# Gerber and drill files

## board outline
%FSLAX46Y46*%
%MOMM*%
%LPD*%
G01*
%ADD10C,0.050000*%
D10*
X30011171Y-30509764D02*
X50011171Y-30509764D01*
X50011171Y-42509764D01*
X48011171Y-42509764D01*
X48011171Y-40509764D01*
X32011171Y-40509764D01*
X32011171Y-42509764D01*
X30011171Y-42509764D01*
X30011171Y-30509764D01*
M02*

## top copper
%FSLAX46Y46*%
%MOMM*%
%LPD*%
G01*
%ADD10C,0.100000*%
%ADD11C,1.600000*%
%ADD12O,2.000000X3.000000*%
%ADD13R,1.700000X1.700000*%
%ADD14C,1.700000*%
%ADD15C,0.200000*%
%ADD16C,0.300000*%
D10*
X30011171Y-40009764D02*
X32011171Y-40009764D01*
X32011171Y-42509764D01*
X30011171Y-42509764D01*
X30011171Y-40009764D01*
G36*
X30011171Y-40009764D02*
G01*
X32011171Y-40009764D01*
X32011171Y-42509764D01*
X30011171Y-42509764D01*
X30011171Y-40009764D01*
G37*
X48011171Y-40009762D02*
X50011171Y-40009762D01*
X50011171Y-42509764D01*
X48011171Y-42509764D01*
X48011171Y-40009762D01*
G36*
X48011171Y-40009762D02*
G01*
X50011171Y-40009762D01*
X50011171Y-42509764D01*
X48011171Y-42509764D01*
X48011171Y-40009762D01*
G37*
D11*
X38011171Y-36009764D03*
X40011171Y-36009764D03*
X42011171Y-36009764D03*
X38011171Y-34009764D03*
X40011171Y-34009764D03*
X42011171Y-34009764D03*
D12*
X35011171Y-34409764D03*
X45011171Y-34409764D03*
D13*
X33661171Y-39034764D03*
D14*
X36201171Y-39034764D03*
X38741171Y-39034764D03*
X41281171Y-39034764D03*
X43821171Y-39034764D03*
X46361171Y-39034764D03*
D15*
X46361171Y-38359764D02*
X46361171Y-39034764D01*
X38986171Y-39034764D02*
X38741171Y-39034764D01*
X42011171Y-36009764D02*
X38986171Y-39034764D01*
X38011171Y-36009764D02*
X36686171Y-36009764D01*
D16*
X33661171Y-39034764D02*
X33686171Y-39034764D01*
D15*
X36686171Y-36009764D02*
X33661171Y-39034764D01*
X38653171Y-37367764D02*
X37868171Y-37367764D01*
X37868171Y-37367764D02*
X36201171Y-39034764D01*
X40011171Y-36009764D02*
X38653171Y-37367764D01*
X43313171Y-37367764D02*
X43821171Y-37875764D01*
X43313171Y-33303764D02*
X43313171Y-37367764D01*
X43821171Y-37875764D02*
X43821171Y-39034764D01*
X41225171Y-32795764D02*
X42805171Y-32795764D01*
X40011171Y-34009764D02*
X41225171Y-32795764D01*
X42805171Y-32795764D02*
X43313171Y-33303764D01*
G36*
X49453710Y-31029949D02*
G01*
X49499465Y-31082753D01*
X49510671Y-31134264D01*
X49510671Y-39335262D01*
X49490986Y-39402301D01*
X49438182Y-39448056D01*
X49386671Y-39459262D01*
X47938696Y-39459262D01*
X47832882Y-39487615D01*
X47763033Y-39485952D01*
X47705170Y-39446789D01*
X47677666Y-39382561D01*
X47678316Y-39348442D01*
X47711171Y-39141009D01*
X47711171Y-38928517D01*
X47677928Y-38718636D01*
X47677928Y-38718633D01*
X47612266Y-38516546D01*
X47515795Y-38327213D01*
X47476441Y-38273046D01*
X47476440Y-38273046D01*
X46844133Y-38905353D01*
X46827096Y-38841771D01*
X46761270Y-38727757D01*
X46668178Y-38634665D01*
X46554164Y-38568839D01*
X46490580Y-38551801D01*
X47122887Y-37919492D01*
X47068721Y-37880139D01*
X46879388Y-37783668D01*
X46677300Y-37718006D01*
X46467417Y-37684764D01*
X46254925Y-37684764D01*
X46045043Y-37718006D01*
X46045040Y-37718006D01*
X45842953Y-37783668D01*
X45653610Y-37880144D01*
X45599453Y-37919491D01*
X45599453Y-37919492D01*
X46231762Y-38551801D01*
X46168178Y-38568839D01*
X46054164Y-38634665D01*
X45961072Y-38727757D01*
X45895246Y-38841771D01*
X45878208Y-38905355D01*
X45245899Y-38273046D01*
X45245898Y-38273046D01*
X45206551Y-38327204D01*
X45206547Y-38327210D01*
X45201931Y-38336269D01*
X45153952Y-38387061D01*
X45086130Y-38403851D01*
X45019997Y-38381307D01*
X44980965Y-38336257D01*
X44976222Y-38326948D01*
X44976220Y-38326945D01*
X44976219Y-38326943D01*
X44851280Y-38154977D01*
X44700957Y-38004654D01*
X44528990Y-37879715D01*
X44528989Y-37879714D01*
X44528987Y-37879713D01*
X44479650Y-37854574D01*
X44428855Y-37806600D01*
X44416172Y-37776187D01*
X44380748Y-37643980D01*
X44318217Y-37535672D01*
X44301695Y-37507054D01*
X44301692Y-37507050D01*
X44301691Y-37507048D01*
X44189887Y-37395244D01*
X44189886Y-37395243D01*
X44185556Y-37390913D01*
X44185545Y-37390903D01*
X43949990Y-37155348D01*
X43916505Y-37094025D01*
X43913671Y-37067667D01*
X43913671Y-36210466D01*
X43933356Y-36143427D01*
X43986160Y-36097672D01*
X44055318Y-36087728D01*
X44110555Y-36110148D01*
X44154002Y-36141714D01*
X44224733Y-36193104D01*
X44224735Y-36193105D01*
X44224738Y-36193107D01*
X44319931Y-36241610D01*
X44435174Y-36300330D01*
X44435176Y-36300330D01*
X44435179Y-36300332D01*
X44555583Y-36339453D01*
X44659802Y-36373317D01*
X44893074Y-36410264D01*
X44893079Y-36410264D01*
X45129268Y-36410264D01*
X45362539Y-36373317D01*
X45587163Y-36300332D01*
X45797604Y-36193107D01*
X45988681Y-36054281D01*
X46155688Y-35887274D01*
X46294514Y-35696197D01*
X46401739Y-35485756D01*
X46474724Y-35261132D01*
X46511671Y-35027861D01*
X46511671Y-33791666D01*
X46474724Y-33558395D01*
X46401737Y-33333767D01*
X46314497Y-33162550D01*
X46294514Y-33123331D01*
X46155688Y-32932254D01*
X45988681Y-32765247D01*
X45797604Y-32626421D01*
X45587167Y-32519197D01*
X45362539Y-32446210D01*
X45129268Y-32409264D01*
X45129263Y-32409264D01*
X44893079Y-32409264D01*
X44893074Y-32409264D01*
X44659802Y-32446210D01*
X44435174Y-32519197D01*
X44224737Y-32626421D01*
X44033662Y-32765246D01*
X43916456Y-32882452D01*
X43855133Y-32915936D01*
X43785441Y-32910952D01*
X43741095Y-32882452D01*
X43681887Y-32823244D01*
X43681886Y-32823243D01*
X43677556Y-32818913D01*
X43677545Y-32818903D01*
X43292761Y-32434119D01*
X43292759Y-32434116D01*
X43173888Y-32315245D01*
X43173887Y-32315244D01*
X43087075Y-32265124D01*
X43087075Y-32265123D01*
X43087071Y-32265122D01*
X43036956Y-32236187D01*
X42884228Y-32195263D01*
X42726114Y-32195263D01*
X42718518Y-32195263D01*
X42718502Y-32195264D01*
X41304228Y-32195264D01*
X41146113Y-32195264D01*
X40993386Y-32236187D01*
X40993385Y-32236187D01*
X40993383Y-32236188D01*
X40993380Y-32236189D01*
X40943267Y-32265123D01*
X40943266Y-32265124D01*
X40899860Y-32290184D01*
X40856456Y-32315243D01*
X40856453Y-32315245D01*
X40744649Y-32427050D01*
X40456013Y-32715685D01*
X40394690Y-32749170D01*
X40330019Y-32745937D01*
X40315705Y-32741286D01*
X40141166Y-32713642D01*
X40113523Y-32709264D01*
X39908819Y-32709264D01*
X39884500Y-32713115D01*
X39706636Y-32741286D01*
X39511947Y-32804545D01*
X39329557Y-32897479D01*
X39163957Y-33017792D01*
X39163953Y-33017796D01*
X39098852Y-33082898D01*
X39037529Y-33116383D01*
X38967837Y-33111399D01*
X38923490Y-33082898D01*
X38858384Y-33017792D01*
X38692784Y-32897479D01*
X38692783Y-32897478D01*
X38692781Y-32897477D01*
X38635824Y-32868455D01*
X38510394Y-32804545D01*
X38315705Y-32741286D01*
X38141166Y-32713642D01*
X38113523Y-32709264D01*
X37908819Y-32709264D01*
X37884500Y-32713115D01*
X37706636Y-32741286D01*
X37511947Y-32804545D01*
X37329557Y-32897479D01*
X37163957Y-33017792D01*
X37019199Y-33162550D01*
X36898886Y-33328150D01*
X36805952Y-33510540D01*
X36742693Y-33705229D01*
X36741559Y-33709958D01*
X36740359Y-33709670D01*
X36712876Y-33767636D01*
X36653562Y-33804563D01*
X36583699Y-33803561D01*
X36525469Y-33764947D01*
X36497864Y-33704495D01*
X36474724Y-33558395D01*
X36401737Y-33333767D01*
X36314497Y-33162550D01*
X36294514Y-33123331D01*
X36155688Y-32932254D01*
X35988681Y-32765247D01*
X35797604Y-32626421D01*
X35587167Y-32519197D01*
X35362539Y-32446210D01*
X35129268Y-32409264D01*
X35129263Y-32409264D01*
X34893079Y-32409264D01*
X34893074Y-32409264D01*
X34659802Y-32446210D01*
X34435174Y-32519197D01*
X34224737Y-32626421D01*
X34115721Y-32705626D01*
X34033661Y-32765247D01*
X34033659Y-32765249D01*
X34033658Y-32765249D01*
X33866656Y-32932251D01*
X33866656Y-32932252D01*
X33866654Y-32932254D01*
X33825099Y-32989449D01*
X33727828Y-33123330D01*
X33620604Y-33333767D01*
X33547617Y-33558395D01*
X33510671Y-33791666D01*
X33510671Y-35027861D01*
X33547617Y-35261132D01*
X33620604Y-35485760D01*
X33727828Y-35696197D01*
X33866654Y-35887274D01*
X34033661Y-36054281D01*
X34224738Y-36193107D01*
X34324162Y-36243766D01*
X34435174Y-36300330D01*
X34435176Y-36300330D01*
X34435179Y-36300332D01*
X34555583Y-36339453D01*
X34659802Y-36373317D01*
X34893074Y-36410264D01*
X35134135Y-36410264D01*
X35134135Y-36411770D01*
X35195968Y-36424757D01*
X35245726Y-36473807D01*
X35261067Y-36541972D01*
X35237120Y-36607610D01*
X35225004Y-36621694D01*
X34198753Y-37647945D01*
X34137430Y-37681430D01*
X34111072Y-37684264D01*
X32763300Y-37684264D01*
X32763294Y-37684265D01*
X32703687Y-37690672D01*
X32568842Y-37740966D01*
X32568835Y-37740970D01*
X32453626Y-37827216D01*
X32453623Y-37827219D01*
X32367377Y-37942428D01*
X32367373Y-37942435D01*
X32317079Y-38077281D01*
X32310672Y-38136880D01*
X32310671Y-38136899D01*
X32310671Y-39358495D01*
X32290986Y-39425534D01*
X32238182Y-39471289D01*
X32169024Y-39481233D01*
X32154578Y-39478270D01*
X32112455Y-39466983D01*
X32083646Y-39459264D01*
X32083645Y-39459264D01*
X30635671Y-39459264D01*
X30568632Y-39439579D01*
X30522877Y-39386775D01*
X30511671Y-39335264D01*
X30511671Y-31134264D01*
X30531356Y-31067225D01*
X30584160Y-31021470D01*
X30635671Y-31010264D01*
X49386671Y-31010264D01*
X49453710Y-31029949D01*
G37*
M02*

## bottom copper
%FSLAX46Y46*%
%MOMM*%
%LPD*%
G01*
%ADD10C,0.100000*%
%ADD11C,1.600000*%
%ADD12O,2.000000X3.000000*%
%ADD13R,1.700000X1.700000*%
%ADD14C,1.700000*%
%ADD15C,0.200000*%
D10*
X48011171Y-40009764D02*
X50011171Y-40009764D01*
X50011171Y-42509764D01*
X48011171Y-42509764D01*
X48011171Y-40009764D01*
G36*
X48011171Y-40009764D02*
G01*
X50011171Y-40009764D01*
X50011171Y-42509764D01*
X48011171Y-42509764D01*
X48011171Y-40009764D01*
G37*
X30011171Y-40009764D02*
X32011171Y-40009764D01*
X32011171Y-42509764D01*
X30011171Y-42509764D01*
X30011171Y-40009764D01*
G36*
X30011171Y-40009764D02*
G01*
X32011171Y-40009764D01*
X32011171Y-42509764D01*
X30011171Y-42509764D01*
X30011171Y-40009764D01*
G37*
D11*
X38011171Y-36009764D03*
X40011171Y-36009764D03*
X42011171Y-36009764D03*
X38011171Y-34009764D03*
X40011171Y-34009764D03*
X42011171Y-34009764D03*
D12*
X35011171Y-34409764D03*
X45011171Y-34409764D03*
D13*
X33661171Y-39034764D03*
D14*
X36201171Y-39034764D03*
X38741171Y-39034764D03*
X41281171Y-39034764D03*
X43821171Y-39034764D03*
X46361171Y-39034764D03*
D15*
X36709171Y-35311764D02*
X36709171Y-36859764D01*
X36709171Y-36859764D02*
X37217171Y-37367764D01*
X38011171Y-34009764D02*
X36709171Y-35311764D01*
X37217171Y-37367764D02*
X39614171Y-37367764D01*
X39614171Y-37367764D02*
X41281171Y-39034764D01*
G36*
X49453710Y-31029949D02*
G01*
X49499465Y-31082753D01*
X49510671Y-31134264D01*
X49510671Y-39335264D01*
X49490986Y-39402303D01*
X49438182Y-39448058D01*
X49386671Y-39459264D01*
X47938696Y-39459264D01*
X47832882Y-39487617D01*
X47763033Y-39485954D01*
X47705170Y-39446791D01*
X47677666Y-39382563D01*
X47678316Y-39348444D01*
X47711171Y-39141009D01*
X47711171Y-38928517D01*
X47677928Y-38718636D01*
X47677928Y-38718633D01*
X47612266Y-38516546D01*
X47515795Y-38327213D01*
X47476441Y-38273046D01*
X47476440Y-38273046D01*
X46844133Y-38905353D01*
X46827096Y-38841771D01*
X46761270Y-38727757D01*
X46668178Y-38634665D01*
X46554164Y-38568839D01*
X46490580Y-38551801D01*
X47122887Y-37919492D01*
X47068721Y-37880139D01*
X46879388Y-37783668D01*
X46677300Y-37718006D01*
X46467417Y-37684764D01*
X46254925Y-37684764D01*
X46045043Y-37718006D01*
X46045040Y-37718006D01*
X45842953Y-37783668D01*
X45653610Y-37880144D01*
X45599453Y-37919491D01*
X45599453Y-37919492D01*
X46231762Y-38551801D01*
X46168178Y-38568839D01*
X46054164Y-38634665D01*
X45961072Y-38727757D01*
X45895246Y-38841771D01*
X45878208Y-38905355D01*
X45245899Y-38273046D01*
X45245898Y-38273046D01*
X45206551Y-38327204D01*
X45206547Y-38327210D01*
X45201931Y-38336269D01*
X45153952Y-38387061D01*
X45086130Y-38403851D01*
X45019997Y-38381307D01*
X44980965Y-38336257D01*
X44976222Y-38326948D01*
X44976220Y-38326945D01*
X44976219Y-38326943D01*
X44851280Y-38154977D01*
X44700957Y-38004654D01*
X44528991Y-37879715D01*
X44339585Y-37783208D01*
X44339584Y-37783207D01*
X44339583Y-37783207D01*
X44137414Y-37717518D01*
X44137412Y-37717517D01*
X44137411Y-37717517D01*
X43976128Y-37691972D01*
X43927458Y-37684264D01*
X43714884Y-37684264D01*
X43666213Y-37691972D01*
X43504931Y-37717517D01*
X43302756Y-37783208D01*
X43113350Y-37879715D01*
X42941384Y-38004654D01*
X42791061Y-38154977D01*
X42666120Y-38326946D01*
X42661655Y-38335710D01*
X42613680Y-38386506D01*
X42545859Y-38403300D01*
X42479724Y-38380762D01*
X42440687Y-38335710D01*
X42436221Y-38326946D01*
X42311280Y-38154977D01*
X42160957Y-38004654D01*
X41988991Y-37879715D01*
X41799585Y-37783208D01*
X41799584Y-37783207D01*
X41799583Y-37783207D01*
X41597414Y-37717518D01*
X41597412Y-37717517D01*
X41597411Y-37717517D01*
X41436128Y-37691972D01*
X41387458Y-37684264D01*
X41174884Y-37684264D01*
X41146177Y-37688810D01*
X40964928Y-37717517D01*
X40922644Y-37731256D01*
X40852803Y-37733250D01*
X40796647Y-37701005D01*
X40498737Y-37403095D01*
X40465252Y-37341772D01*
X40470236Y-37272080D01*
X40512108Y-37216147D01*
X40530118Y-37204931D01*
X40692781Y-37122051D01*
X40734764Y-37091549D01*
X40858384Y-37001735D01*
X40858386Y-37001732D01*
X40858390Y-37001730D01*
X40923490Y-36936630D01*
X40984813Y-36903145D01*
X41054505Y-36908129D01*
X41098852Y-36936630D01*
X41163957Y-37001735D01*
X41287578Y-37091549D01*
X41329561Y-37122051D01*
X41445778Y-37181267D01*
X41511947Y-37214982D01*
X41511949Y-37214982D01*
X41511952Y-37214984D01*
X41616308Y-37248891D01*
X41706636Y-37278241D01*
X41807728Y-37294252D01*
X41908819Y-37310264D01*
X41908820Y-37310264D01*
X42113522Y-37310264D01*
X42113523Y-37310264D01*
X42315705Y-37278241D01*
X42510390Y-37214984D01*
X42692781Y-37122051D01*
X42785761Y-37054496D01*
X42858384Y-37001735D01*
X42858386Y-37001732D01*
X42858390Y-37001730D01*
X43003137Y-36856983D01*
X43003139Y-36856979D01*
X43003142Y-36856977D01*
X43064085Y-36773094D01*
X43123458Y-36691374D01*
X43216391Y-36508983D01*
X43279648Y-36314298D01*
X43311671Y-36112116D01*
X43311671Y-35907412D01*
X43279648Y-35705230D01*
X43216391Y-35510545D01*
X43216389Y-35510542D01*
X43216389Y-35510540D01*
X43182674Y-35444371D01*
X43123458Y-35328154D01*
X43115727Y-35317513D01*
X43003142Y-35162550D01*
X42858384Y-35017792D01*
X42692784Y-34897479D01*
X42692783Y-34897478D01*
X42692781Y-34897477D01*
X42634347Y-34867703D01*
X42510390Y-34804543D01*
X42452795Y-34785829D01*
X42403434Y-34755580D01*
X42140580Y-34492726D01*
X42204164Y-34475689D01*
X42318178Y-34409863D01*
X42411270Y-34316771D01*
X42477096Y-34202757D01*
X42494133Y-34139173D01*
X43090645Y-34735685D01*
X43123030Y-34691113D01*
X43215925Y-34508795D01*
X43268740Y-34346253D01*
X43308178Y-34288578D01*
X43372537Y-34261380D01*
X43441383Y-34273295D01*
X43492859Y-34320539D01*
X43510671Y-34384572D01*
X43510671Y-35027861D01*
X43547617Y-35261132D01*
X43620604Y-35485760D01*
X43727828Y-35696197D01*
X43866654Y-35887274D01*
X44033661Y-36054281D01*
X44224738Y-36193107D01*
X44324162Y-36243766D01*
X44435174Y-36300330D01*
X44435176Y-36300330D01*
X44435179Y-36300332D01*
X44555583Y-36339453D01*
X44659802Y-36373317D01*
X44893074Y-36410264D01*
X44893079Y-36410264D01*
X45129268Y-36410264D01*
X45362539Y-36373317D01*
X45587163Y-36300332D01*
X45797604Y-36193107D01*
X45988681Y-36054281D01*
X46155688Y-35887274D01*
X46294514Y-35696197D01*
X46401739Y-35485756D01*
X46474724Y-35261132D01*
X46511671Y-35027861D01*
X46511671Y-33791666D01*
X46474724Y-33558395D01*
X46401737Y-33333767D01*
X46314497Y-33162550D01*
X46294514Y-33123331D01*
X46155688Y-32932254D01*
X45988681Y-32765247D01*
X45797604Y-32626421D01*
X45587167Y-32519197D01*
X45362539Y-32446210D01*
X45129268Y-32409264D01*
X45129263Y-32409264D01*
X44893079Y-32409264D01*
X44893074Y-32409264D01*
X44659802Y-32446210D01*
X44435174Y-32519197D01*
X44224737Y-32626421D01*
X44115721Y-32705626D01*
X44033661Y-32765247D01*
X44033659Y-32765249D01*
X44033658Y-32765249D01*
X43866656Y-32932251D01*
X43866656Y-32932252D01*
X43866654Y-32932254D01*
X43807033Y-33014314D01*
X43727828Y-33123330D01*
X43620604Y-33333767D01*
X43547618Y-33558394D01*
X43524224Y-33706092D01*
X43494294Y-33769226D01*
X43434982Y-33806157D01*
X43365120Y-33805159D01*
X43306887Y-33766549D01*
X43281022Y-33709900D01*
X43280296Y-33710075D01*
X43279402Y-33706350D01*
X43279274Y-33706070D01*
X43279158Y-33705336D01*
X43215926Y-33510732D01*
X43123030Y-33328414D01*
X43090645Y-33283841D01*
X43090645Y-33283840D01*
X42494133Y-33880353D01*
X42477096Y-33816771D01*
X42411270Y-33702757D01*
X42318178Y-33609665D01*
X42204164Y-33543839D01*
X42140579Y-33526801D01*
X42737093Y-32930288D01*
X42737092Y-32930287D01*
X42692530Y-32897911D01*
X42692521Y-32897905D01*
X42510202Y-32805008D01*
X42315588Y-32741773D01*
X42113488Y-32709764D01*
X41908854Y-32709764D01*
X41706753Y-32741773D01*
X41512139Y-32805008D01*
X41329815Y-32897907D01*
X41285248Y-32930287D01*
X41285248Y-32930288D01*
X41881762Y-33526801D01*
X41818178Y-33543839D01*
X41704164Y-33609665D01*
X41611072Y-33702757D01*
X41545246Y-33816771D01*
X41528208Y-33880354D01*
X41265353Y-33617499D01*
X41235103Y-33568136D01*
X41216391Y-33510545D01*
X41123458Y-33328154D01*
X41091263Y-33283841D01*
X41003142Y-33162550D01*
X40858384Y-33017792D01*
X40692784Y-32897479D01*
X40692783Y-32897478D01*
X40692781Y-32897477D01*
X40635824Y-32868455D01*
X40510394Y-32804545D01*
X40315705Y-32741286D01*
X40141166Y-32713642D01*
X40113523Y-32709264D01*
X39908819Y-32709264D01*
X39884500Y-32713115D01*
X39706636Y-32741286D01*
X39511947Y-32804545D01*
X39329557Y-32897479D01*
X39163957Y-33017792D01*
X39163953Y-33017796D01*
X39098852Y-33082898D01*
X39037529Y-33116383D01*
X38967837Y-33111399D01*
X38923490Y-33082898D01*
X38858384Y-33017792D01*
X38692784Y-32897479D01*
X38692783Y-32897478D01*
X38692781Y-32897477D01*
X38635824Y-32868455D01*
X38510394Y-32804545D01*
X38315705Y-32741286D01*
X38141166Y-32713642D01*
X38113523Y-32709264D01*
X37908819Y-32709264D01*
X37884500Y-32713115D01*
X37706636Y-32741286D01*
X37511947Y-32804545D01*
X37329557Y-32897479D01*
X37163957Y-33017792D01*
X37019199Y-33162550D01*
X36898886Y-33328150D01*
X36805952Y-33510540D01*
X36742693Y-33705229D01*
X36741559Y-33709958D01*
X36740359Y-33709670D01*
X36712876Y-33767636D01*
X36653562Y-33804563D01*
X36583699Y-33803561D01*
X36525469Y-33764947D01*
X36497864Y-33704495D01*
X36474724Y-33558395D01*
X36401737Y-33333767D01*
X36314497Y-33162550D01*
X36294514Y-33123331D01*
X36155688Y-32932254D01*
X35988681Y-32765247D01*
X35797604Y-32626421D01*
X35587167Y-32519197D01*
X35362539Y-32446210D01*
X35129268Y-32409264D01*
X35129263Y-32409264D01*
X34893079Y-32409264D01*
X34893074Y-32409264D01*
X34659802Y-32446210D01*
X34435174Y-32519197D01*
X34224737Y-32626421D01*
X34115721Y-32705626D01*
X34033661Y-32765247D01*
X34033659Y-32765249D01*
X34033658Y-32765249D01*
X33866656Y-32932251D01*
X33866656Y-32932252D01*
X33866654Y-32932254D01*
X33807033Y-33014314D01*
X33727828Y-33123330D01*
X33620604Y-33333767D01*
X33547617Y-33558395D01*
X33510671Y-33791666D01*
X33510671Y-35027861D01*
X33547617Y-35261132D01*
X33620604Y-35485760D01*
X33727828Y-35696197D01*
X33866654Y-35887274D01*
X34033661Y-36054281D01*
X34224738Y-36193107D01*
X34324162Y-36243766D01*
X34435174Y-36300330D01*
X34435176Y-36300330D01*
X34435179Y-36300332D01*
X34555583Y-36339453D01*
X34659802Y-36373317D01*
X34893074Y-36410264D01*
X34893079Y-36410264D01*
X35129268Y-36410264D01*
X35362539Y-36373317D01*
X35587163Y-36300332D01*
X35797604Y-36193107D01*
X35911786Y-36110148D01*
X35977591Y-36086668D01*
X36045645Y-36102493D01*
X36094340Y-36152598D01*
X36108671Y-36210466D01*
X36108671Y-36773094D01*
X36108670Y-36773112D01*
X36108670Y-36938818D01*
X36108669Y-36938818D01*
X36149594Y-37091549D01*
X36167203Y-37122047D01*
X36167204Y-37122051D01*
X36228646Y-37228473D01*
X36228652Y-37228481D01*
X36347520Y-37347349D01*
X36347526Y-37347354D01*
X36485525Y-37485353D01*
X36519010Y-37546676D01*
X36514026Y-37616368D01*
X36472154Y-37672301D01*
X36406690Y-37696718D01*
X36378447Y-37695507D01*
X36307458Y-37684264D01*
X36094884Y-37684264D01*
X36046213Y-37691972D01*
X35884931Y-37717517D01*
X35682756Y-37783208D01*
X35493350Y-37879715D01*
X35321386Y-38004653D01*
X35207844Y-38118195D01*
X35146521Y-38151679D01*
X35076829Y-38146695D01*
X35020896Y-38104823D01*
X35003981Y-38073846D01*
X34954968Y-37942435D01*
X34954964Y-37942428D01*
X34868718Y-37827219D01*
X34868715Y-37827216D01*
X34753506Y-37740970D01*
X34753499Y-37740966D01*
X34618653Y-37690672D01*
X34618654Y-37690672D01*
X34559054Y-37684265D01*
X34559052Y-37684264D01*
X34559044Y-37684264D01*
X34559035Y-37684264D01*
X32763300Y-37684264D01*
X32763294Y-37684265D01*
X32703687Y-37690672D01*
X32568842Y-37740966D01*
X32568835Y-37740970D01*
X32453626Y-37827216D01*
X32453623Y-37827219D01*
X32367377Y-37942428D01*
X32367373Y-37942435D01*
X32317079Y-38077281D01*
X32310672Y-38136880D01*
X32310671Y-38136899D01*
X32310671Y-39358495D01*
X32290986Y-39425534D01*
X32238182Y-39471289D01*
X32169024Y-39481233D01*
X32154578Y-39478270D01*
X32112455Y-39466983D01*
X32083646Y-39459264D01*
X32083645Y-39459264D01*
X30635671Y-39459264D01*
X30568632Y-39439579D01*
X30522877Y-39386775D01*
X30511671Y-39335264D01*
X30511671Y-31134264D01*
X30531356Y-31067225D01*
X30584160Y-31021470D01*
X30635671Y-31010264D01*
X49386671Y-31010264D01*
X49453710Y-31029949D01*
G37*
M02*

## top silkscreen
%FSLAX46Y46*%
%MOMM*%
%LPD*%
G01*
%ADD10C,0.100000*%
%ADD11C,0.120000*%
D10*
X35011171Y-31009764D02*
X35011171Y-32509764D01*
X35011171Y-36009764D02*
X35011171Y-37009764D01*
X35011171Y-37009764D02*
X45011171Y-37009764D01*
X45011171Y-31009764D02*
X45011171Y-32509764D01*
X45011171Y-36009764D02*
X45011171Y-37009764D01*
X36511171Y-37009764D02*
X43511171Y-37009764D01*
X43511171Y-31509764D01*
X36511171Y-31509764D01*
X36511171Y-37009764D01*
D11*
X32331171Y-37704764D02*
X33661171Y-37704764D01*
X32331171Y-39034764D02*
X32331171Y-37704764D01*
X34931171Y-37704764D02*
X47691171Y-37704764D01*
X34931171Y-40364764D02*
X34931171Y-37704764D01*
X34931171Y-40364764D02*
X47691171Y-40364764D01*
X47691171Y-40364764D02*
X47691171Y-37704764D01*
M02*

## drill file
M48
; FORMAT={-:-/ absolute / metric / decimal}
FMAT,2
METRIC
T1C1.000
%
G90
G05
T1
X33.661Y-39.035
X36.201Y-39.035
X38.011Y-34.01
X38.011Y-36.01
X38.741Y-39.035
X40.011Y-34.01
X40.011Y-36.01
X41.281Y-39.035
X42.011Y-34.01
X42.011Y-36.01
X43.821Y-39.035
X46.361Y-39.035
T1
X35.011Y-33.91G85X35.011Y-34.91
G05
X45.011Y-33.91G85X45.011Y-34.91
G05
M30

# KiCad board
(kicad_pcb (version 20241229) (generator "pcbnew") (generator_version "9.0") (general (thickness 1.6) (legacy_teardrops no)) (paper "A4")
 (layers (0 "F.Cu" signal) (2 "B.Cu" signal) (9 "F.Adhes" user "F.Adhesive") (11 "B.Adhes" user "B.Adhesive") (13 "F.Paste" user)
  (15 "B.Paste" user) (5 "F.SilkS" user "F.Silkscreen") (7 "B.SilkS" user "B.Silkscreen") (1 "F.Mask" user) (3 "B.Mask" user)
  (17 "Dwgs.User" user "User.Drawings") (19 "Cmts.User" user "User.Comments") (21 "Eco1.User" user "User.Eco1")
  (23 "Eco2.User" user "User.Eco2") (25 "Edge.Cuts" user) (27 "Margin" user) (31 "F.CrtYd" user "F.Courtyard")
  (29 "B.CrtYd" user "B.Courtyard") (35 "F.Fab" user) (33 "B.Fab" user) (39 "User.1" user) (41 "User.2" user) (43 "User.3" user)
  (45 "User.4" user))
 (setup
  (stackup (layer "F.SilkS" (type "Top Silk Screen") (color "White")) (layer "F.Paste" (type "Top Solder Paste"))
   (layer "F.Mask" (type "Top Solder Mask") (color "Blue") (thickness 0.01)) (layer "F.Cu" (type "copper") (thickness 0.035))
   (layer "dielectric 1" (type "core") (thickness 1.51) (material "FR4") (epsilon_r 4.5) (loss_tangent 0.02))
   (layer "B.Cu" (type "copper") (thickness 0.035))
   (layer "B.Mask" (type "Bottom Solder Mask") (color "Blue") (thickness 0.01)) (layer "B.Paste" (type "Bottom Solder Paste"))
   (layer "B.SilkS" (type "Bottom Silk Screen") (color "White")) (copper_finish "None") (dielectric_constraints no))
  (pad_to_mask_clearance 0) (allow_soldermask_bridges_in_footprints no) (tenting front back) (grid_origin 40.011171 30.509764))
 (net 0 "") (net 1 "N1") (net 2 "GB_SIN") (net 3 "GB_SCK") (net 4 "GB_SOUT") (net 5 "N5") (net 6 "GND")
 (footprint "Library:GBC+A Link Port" (layer "F.Cu") (at 40.011171 35.009764)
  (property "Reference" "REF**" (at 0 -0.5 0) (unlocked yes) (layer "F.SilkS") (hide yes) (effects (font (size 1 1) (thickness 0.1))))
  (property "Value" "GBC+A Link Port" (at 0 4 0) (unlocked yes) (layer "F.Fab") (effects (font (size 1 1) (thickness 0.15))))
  (fp_line (start -5 -4) (end -5 -2.5) (stroke (width 0.1) (type default)) (layer "F.SilkS"))
  (fp_line (start -5 1) (end -5 2) (stroke (width 0.1) (type default)) (layer "F.SilkS"))
  (fp_line (start -5 2) (end 5 2) (stroke (width 0.1) (type default)) (layer "F.SilkS"))
  (fp_line (start 5 -4) (end 5 -2.5) (stroke (width 0.1) (type default)) (layer "F.SilkS"))
  (fp_line (start 5 1) (end 5 2) (stroke (width 0.1) (type default)) (layer "F.SilkS"))
  (fp_poly (pts (xy -3.5 2) (xy 3.5 2) (xy 3.5 -3.5) (xy -3.5 -3.5)) (stroke (width 0.1) (type solid)) (fill no) (layer "F.SilkS"))
  (pad "1" thru_hole circle (at -2 1) (size 1.6 1.6) (drill 1) (layers "*.Cu" "*.Mask") (remove_unused_layers no) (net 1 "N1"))
  (pad "2" thru_hole circle (at 0 1) (size 1.6 1.6) (drill 1) (layers "*.Cu" "*.Mask") (remove_unused_layers no) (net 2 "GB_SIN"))
  (pad "3" thru_hole circle (at 2 1) (size 1.6 1.6) (drill 1) (layers "*.Cu" "*.Mask") (remove_unused_layers no) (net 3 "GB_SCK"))
  (pad "4" thru_hole circle (at -2 -1) (size 1.6 1.6) (drill 1) (layers "*.Cu" "*.Mask") (remove_unused_layers no) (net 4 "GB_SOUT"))
  (pad "5" thru_hole circle (at 0 -1) (size 1.6 1.6) (drill 1) (layers "*.Cu" "*.Mask") (remove_unused_layers no) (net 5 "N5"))
  (pad "6" thru_hole circle (at 2 -1) (size 1.6 1.6) (drill 1) (layers "*.Cu" "*.Mask") (remove_unused_layers no) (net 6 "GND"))
  (pad "MP" thru_hole oval (at -5 -0.6) (size 2 3) (drill oval 1 2) (layers "*.Cu" "*.Mask") (remove_unused_layers no)
   (thermal_bridge_angle 45))
  (pad "MP" thru_hole oval (at 5 -0.6) (size 2 3) (drill oval 1 2) (layers "*.Cu" "*.Mask") (remove_unused_layers no)
   (thermal_bridge_angle 45)))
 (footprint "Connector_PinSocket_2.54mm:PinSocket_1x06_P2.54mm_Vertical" (layer "F.Cu") (at 33.661171 39.034764 90)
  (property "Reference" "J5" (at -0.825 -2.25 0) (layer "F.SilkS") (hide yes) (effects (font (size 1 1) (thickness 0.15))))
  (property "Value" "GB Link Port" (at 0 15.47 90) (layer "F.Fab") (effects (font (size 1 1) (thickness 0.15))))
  (fp_line (start 1.33 -1.33) (end 1.33 0) (stroke (width 0.12) (type solid)) (layer "F.SilkS"))
  (fp_line (start 0 -1.33) (end 1.33 -1.33) (stroke (width 0.12) (type solid)) (layer "F.SilkS"))
  (fp_line (start 1.33 1.27) (end 1.33 14.03) (stroke (width 0.12) (type solid)) (layer "F.SilkS"))
  (fp_line (start -1.33 1.27) (end 1.33 1.27) (stroke (width 0.12) (type solid)) (layer "F.SilkS"))
  (fp_line (start -1.33 1.27) (end -1.33 14.03) (stroke (width 0.12) (type solid)) (layer "F.SilkS"))
  (fp_line (start -1.33 14.03) (end 1.33 14.03) (stroke (width 0.12) (type solid)) (layer "F.SilkS"))
  (pad "1" thru_hole rect (at 0 0 90) (size 1.7 1.7) (drill 1) (layers "*.Cu" "*.Mask") (remove_unused_layers no) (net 1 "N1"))
  (pad "2" thru_hole circle (at 0 2.54 90) (size 1.7 1.7) (drill 1) (layers "*.Cu" "*.Mask") (remove_unused_layers no) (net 2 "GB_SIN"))
  (pad "3" thru_hole circle (at 0 5.08 90) (size 1.7 1.7) (drill 1) (layers "*.Cu" "*.Mask") (remove_unused_layers no) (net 3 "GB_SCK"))
  (pad "4" thru_hole circle (at 0 7.62 90) (size 1.7 1.7) (drill 1) (layers "*.Cu" "*.Mask") (remove_unused_layers no) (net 4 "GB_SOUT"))
  (pad "5" thru_hole circle (at 0 10.16 90) (size 1.7 1.7) (drill 1) (layers "*.Cu" "*.Mask") (remove_unused_layers no) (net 5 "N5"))
  (pad "6" thru_hole circle (at 0 12.7 90) (size 1.7 1.7) (drill 1) (layers "*.Cu" "*.Mask") (remove_unused_layers no) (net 6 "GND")))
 (gr_rect (start 30.011171 40.009764) (end 32.011171 42.509764) (stroke (width 0.1) (type solid)) (fill yes) (layer "F.Cu"))
 (gr_rect (start 48.011171 40.009762) (end 50.011171 42.509764) (stroke (width 0.1) (type solid)) (fill yes) (layer "F.Cu"))
 (gr_rect (start 48.011171 40.009764) (end 50.011171 42.509764) (stroke (width 0.1) (type solid)) (fill yes) (layer "B.Cu"))
 (gr_rect (start 30.011171 40.009764) (end 32.011171 42.509764) (stroke (width 0.1) (type solid)) (fill yes) (layer "B.Cu"))
 (gr_poly
  (pts (xy 30.011171 30.509764) (xy 50.011171 30.509764) (xy 50.011171 42.509764) (xy 48.011171 42.509764) (xy 48.011171 40.509764)
   (xy 32.011171 40.509764) (xy 32.011171 42.509764) (xy 30.011171 42.509764))
  (stroke (width 0.05) (type solid)) (fill no) (layer "Edge.Cuts"))
 (segment (start 46.361171 38.359764) (end 46.361171 39.034764) (width 0.2) (layer "F.Cu") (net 6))
 (segment (start 38.986171 39.034764) (end 38.741171 39.034764) (width 0.2) (layer "F.Cu") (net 3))
 (segment (start 42.011171 36.009764) (end 38.986171 39.034764) (width 0.2) (layer "F.Cu") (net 3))
 (segment (start 38.011171 36.009764) (end 36.686171 36.009764) (width 0.2) (layer "F.Cu") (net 1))
 (segment (start 33.661171 39.034764) (end 33.686171 39.034764) (width 0.3) (layer "F.Cu") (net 1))
 (segment (start 36.686171 36.009764) (end 33.661171 39.034764) (width 0.2) (layer "F.Cu") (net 1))
 (segment (start 38.653171 37.367764) (end 37.868171 37.367764) (width 0.2) (layer "F.Cu") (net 2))
 (segment (start 37.868171 37.367764) (end 36.201171 39.034764) (width 0.2) (layer "F.Cu") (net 2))
 (segment (start 40.011171 36.009764) (end 38.653171 37.367764) (width 0.2) (layer "F.Cu") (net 2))
 (segment (start 43.313171 37.367764) (end 43.821171 37.875764) (width 0.2) (layer "F.Cu") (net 5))
 (segment (start 43.313171 33.303764) (end 43.313171 37.367764) (width 0.2) (layer "F.Cu") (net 5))
 (segment (start 43.821171 37.875764) (end 43.821171 39.034764) (width 0.2) (layer "F.Cu") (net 5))
 (segment (start 41.225171 32.795764) (end 42.805171 32.795764) (width 0.2) (layer "F.Cu") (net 5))
 (segment (start 40.011171 34.009764) (end 41.225171 32.795764) (width 0.2) (layer "F.Cu") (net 5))
 (segment (start 42.805171 32.795764) (end 43.313171 33.303764) (width 0.2) (layer "F.Cu") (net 5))
 (segment (start 36.709171 35.311764) (end 36.709171 36.859764) (width 0.2) (layer "B.Cu") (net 4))
 (segment (start 36.709171 36.859764) (end 37.217171 37.367764) (width 0.2) (layer "B.Cu") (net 4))
 (segment (start 38.011171 34.009764) (end 36.709171 35.311764) (width 0.2) (layer "B.Cu") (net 4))
 (segment (start 37.217171 37.367764) (end 39.614171 37.367764) (width 0.2) (layer "B.Cu") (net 4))
 (segment (start 39.614171 37.367764) (end 41.281171 39.034764) (width 0.2) (layer "B.Cu") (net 4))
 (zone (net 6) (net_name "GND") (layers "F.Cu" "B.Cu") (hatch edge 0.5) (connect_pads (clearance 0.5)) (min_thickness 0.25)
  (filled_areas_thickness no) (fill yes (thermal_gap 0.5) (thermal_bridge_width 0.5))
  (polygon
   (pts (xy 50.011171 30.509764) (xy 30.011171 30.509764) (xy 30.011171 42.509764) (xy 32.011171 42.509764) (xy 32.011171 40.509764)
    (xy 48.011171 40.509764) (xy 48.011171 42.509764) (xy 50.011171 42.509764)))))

